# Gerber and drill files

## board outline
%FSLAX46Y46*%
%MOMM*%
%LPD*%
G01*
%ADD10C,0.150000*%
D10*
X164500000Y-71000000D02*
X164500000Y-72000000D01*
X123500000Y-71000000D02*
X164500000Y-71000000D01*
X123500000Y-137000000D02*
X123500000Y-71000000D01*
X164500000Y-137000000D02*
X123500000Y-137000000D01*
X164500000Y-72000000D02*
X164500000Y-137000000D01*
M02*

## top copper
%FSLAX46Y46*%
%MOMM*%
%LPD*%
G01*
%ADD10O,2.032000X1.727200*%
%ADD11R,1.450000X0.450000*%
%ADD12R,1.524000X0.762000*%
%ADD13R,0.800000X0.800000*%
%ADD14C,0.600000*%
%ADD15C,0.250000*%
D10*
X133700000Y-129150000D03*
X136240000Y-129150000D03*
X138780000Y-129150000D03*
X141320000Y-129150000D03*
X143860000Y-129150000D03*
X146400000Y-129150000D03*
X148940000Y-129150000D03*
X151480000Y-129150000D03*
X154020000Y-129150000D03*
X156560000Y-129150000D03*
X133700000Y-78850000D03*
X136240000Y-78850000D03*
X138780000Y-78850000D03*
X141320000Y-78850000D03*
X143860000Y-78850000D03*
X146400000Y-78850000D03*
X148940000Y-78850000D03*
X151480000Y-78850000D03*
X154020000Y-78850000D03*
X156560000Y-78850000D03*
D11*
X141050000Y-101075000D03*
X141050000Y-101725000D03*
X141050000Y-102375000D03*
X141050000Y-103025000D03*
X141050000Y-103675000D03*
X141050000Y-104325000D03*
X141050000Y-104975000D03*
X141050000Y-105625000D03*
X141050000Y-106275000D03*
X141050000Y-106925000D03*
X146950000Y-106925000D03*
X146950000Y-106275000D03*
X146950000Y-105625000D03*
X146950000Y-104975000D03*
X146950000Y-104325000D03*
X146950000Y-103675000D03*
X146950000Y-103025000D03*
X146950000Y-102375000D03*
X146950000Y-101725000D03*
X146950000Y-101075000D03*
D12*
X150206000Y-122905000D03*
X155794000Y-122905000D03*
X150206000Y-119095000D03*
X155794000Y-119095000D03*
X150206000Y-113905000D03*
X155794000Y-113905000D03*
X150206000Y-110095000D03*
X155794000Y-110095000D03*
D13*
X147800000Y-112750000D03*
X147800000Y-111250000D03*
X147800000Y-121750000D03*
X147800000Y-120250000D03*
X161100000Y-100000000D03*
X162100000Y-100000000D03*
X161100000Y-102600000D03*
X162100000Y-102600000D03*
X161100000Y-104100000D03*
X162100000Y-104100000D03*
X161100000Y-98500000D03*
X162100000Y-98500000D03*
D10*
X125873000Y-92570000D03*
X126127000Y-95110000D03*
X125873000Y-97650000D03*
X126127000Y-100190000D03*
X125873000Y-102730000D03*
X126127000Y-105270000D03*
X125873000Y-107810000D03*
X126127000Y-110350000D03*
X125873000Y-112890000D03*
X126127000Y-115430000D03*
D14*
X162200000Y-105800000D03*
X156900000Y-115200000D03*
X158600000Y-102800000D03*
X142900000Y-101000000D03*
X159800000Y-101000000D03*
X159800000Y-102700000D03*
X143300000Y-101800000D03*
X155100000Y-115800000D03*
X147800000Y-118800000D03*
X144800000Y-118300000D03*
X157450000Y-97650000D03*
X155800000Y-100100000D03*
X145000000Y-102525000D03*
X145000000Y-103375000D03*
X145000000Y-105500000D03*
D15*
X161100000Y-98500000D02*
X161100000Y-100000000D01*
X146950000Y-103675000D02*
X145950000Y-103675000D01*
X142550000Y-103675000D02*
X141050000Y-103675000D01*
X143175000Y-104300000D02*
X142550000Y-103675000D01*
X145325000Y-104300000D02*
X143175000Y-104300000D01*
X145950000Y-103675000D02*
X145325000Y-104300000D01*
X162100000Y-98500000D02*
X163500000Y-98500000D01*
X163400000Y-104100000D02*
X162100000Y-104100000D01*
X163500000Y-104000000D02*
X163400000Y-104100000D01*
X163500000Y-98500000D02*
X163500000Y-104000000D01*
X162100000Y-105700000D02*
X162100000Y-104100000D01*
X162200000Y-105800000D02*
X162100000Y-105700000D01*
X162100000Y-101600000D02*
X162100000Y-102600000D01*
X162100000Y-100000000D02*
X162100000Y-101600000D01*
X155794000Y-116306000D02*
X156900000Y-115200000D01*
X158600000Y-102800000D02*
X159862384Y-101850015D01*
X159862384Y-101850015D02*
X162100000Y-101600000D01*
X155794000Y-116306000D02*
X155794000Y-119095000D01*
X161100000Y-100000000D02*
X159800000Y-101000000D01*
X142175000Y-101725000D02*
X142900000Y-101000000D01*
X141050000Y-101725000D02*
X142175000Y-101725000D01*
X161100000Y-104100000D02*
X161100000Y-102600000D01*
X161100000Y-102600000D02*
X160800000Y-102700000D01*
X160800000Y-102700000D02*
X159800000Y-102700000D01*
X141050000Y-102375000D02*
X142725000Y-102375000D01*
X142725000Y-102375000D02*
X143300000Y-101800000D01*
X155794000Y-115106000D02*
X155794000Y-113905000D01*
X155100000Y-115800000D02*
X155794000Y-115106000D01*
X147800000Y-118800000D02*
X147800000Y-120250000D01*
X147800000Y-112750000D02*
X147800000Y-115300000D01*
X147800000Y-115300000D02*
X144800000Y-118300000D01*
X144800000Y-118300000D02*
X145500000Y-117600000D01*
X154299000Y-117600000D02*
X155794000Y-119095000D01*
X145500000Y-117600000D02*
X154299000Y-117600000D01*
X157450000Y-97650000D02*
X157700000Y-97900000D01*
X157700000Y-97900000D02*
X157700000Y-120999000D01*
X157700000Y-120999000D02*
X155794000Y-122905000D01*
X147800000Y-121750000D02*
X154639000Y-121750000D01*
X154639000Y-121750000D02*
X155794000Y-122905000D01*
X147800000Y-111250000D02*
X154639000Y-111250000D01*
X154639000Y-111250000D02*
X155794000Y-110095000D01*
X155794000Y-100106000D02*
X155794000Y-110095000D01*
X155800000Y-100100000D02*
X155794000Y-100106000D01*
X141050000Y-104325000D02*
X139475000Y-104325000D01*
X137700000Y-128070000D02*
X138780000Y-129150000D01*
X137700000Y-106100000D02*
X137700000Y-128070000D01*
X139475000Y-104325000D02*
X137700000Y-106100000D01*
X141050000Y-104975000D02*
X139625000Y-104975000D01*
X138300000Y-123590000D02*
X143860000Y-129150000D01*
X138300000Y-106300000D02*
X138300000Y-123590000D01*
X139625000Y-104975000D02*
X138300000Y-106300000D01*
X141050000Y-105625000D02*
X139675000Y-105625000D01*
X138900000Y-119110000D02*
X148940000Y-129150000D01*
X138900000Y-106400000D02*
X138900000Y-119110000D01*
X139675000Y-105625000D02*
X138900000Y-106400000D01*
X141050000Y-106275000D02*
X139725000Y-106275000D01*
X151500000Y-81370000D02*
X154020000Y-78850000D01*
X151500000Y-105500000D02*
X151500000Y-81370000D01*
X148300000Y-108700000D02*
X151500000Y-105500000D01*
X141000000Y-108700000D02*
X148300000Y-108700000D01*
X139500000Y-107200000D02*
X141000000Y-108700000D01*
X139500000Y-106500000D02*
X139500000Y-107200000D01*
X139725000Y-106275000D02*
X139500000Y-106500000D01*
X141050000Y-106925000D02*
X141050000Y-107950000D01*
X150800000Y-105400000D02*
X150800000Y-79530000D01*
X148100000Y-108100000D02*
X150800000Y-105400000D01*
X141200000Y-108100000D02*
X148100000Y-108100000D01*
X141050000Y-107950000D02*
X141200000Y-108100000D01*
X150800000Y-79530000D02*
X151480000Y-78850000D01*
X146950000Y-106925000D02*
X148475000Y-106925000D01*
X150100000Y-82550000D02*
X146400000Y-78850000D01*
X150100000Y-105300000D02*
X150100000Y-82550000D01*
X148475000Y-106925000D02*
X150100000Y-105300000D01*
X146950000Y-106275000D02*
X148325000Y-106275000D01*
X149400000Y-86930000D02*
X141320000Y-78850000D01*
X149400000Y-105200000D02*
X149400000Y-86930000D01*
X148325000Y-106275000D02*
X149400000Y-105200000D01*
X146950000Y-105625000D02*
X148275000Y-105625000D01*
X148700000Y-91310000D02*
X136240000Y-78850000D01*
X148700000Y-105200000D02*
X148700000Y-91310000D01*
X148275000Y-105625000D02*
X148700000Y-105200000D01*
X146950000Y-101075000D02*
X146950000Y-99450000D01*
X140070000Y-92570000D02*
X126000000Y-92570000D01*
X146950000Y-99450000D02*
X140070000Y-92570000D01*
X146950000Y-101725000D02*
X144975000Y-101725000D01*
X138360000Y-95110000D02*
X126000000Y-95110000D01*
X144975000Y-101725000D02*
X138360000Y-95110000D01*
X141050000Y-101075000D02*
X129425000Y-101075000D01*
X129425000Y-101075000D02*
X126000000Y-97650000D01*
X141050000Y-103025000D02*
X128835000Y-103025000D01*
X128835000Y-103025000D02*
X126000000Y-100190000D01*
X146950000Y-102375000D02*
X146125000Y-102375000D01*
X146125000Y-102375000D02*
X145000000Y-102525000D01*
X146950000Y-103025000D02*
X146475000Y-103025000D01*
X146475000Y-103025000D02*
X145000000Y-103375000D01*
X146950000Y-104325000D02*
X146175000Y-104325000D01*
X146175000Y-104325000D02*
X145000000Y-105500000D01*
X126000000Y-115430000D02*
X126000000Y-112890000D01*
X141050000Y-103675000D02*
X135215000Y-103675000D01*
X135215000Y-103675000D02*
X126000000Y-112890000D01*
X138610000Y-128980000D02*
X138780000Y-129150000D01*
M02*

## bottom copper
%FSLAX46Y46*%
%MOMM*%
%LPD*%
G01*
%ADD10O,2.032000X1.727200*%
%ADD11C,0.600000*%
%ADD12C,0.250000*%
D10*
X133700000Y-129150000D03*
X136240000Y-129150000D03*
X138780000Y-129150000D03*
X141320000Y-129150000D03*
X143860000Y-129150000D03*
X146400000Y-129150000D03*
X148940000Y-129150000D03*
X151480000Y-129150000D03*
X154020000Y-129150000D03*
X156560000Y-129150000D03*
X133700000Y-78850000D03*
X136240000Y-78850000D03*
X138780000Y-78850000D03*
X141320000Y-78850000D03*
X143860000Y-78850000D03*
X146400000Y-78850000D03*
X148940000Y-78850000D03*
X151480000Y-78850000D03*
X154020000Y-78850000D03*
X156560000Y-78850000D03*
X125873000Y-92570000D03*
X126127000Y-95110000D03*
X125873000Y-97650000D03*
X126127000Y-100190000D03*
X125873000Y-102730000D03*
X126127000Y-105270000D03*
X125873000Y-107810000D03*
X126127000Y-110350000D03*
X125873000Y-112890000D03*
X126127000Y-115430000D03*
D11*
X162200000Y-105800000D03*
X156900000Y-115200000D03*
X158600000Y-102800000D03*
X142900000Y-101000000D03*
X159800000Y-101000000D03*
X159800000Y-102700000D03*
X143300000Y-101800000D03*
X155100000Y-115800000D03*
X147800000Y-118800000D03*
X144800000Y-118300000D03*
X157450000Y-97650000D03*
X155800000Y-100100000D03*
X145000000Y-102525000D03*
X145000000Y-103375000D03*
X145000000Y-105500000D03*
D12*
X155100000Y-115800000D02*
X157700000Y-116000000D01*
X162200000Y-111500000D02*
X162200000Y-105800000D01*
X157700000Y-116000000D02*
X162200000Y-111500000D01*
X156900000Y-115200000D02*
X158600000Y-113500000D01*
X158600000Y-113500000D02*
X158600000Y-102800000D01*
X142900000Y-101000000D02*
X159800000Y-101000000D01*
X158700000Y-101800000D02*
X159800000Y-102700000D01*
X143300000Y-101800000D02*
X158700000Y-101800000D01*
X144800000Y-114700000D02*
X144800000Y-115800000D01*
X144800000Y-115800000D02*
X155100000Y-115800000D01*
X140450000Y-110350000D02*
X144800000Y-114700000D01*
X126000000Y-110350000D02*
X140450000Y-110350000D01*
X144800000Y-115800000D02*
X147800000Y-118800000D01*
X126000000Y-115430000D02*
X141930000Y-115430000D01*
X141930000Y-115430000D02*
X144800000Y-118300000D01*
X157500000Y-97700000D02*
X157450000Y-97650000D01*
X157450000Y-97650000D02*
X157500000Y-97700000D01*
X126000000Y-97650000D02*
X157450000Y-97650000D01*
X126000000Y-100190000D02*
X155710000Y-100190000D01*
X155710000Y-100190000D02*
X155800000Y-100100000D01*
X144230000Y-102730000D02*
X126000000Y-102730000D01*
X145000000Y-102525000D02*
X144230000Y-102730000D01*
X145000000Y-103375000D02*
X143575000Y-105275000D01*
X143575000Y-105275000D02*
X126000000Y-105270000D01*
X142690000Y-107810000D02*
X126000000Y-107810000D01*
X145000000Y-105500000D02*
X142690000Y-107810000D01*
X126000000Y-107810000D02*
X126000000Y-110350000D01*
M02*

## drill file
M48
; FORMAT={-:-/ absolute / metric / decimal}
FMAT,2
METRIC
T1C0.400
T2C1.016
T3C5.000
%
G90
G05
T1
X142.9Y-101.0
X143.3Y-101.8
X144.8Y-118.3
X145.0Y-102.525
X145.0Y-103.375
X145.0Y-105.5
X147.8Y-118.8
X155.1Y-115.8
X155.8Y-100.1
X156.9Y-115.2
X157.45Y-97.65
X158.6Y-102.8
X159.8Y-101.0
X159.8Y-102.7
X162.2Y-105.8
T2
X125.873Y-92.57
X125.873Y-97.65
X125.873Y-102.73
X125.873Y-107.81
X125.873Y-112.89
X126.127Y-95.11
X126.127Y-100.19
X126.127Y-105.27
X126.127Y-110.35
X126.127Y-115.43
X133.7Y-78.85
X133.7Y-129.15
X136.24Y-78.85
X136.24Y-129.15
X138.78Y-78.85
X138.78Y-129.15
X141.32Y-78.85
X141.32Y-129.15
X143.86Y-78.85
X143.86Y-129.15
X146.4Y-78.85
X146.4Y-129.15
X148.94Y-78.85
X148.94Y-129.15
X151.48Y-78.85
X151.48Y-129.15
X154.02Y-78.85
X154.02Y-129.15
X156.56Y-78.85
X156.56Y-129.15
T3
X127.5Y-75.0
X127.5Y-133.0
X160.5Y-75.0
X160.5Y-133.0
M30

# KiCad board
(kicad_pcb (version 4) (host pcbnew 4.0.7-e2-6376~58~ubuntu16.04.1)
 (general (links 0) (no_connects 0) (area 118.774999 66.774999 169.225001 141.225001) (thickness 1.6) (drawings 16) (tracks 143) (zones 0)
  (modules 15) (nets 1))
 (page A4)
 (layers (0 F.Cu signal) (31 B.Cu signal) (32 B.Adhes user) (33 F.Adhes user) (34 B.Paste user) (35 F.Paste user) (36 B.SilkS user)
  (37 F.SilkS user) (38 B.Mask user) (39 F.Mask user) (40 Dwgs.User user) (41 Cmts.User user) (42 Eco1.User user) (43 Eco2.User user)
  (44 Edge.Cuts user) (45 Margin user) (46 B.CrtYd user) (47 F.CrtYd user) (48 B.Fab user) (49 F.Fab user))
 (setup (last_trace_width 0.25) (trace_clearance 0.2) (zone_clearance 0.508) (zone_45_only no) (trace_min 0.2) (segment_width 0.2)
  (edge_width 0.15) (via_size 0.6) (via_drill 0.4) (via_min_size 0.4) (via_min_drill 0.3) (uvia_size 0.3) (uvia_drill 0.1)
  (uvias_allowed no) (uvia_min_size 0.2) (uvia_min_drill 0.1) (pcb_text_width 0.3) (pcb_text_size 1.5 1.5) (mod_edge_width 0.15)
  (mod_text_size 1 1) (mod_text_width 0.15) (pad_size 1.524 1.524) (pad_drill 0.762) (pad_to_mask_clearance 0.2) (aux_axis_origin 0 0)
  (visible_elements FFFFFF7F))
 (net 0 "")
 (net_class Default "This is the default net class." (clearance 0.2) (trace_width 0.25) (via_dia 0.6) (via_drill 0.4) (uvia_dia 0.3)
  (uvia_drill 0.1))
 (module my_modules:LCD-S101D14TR (layer B.Cu) (at 144 104 180)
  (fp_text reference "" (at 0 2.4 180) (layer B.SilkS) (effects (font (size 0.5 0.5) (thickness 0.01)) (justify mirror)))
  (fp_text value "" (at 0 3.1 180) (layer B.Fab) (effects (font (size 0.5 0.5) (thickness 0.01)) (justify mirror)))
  (pad 10 thru_hole oval (at 10.3 -25.15 180) (size 2.032 1.7272) (drill 1.016) (layers *.Cu *.Mask B.SilkS))
  (pad 9 thru_hole oval (at 7.76 -25.15 180) (size 2.032 1.7272) (drill 1.016) (layers *.Cu *.Mask B.SilkS))
  (pad 8 thru_hole oval (at 5.22 -25.15 180) (size 2.032 1.7272) (drill 1.016) (layers *.Cu *.Mask B.SilkS))
  (pad 7 thru_hole oval (at 2.68 -25.15 180) (size 2.032 1.7272) (drill 1.016) (layers *.Cu *.Mask B.SilkS))
  (pad 6 thru_hole oval (at 0.14 -25.15 180) (size 2.032 1.7272) (drill 1.016) (layers *.Cu *.Mask B.SilkS))
  (pad 5 thru_hole oval (at -2.4 -25.15 180) (size 2.032 1.7272) (drill 1.016) (layers *.Cu *.Mask B.SilkS))
  (pad 4 thru_hole oval (at -4.94 -25.15 180) (size 2.032 1.7272) (drill 1.016) (layers *.Cu *.Mask B.SilkS))
  (pad 3 thru_hole oval (at -7.48 -25.15 180) (size 2.032 1.7272) (drill 1.016) (layers *.Cu *.Mask B.SilkS))
  (pad 2 thru_hole oval (at -10.02 -25.15 180) (size 2.032 1.7272) (drill 1.016) (layers *.Cu *.Mask B.SilkS))
  (pad 1 thru_hole oval (at -12.56 -25.15 180) (size 2.032 1.7272) (drill 1.016) (layers *.Cu *.Mask B.SilkS))
  (pad 11 thru_hole oval (at 10.3 25.15 180) (size 2.032 1.7272) (drill 1.016) (layers *.Cu *.Mask B.SilkS))
  (pad 12 thru_hole oval (at 7.76 25.15 180) (size 2.032 1.7272) (drill 1.016) (layers *.Cu *.Mask B.SilkS))
  (pad 13 thru_hole oval (at 5.22 25.15 180) (size 2.032 1.7272) (drill 1.016) (layers *.Cu *.Mask B.SilkS))
  (pad 14 thru_hole oval (at 2.68 25.15 180) (size 2.032 1.7272) (drill 1.016) (layers *.Cu *.Mask B.SilkS))
  (pad 15 thru_hole oval (at 0.14 25.15 180) (size 2.032 1.7272) (drill 1.016) (layers *.Cu *.Mask B.SilkS))
  (pad 16 thru_hole oval (at -2.4 25.15 180) (size 2.032 1.7272) (drill 1.016) (layers *.Cu *.Mask B.SilkS))
  (pad 17 thru_hole oval (at -4.94 25.15 180) (size 2.032 1.7272) (drill 1.016) (layers *.Cu *.Mask B.SilkS))
  (pad 18 thru_hole oval (at -7.48 25.15 180) (size 2.032 1.7272) (drill 1.016) (layers *.Cu *.Mask B.SilkS))
  (pad 19 thru_hole oval (at -10.02 25.15 180) (size 2.032 1.7272) (drill 1.016) (layers *.Cu *.Mask B.SilkS))
  (pad 20 thru_hole oval (at -12.56 25.15 180) (size 2.032 1.7272) (drill 1.016) (layers *.Cu *.Mask B.SilkS)))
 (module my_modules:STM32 (layer F.Cu) (at 144 104)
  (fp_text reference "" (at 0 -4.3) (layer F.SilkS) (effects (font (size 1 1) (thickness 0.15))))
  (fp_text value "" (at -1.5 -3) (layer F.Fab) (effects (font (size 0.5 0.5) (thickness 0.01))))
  (pad BOOT smd rect (at -2.95 -2.925) (size 1.45 0.45) (layers F.Cu F.Paste F.Mask))
  (pad 2 smd rect (at -2.95 -2.275) (size 1.45 0.45) (layers F.Cu F.Paste F.Mask))
  (pad 3 smd rect (at -2.95 -1.625) (size 1.45 0.45) (layers F.Cu F.Paste F.Mask))
  (pad NRST smd rect (at -2.95 -0.975) (size 1.45 0.45) (layers F.Cu F.Paste F.Mask))
  (pad VCC smd rect (at -2.95 -0.325) (size 1.45 0.45) (layers F.Cu F.Paste F.Mask))
  (pad PA0 smd rect (at -2.95 0.325) (size 1.45 0.45) (layers F.Cu F.Paste F.Mask))
  (pad PA1 smd rect (at -2.95 0.975) (size 1.45 0.45) (layers F.Cu F.Paste F.Mask))
  (pad PA2 smd rect (at -2.95 1.625) (size 1.45 0.45) (layers F.Cu F.Paste F.Mask))
  (pad PA3 smd rect (at -2.95 2.275) (size 1.45 0.45) (layers F.Cu F.Paste F.Mask))
  (pad PA4 smd rect (at -2.95 2.925) (size 1.45 0.45) (layers F.Cu F.Paste F.Mask))
  (pad PA5 smd rect (at 2.95 2.925) (size 1.45 0.45) (layers F.Cu F.Paste F.Mask))
  (pad PA6 smd rect (at 2.95 2.275) (size 1.45 0.45) (layers F.Cu F.Paste F.Mask))
  (pad PA7 smd rect (at 2.95 1.625) (size 1.45 0.45) (layers F.Cu F.Paste F.Mask))
  (pad PB1 smd rect (at 2.95 0.975) (size 1.45 0.45) (layers F.Cu F.Paste F.Mask))
  (pad GND smd rect (at 2.95 0.325) (size 1.45 0.45) (layers F.Cu F.Paste F.Mask))
  (pad VCC smd rect (at 2.95 -0.325) (size 1.45 0.45) (layers F.Cu F.Paste F.Mask))
  (pad TX smd rect (at 2.95 -0.975) (size 1.45 0.45) (layers F.Cu F.Paste F.Mask))
  (pad RX smd rect (at 2.95 -1.625) (size 1.45 0.45) (layers F.Cu F.Paste F.Mask))
  (pad DIO smd rect (at 2.95 -2.275) (size 1.45 0.45) (layers F.Cu F.Paste F.Mask))
  (pad CLK smd rect (at 2.95 -2.925) (size 1.45 0.45) (layers F.Cu F.Paste F.Mask)))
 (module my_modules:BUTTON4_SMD (layer F.Cu) (at 153 121)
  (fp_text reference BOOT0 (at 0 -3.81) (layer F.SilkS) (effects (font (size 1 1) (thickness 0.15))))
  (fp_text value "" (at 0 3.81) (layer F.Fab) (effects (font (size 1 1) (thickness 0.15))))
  (pad 1 smd rect (at -2.794 1.905) (size 1.524 0.762) (layers F.Cu F.Paste F.Mask))
  (pad 2 smd rect (at 2.794 1.905) (size 1.524 0.762) (layers F.Cu F.Paste F.Mask))
  (pad 3 smd rect (at -2.794 -1.905) (size 1.524 0.762) (layers F.Cu F.Paste F.Mask))
  (pad 4 smd rect (at 2.794 -1.905) (size 1.524 0.762) (layers F.Cu F.Paste F.Mask)))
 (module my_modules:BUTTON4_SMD (layer F.Cu) (at 153 112)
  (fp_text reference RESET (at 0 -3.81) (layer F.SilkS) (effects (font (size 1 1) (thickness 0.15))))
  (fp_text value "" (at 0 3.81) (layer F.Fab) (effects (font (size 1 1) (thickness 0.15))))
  (pad 1 smd rect (at -2.794 1.905) (size 1.524 0.762) (layers F.Cu F.Paste F.Mask))
  (pad 2 smd rect (at 2.794 1.905) (size 1.524 0.762) (layers F.Cu F.Paste F.Mask))
  (pad 3 smd rect (at -2.794 -1.905) (size 1.524 0.762) (layers F.Cu F.Paste F.Mask))
  (pad 4 smd rect (at 2.794 -1.905) (size 1.524 0.762) (layers F.Cu F.Paste F.Mask)))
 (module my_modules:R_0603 (layer F.Cu) (at 147.8 112 90)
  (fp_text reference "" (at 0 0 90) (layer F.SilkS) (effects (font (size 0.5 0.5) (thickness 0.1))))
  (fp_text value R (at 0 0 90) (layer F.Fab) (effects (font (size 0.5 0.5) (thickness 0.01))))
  (pad 1 smd rect (at -0.75 0 90) (size 0.8 0.8) (layers F.Cu F.Paste F.Mask))
  (pad 2 smd rect (at 0.75 0 90) (size 0.8 0.8) (layers F.Cu F.Paste F.Mask)))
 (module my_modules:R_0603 (layer F.Cu) (at 147.8 121 90)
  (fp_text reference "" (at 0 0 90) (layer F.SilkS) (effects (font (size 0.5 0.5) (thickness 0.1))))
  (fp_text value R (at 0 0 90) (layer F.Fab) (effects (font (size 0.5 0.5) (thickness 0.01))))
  (pad 1 smd rect (at -0.75 0 90) (size 0.8 0.8) (layers F.Cu F.Paste F.Mask))
  (pad 2 smd rect (at 0.75 0 90) (size 0.8 0.8) (layers F.Cu F.Paste F.Mask)))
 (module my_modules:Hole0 (layer F.Cu) (at 160.5 133)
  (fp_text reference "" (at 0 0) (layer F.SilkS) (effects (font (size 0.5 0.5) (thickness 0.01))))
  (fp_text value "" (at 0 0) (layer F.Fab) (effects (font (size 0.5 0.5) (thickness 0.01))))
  (pad "" np_thru_hole circle (at 0 0) (size 5 5) (drill 5) (layers *.Cu *.Mask F.SilkS)))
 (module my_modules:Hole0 (layer F.Cu) (at 127.5 133)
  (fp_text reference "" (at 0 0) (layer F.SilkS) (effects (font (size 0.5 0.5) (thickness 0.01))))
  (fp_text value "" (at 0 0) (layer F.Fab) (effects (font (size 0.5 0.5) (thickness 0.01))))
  (pad "" np_thru_hole circle (at 0 0) (size 5 5) (drill 5) (layers *.Cu *.Mask F.SilkS)))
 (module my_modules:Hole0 (layer F.Cu) (at 160.5 75)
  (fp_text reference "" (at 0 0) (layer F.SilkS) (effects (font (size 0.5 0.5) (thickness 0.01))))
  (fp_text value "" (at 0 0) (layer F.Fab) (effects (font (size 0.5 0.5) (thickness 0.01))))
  (pad "" np_thru_hole circle (at 0 0) (size 5 5) (drill 5) (layers *.Cu *.Mask F.SilkS)))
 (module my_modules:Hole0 (layer F.Cu) (at 127.5 75)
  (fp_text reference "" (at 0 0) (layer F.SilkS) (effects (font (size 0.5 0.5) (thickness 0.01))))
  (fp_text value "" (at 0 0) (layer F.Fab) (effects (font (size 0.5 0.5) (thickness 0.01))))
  (pad "" np_thru_hole circle (at 0 0) (size 5 5) (drill 5) (layers *.Cu *.Mask F.SilkS)))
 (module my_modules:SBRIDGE (layer F.Cu) (at 161.6 100)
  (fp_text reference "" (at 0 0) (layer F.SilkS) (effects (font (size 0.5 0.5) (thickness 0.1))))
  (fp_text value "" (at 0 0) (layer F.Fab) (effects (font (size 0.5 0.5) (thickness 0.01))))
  (pad 1 smd rect (at -0.5 0) (size 0.8 0.8) (layers F.Cu F.Paste F.Mask))
  (pad 2 smd rect (at 0.5 0) (size 0.8 0.8) (layers F.Cu F.Paste F.Mask)))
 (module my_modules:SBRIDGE (layer F.Cu) (at 161.6 102.6)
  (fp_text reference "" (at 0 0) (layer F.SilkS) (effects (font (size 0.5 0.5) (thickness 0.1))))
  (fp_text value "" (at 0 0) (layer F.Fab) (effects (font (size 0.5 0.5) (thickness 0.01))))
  (pad 1 smd rect (at -0.5 0) (size 0.8 0.8) (layers F.Cu F.Paste F.Mask))
  (pad 2 smd rect (at 0.5 0) (size 0.8 0.8) (layers F.Cu F.Paste F.Mask)))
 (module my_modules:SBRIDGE (layer F.Cu) (at 161.6 104.1)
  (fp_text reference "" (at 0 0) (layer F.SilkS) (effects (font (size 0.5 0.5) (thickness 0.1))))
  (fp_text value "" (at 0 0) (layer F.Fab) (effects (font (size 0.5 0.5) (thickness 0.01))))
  (pad 1 smd rect (at -0.5 0) (size 0.8 0.8) (layers F.Cu F.Paste F.Mask))
  (pad 2 smd rect (at 0.5 0) (size 0.8 0.8) (layers F.Cu F.Paste F.Mask)))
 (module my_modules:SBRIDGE (layer F.Cu) (at 161.6 98.5)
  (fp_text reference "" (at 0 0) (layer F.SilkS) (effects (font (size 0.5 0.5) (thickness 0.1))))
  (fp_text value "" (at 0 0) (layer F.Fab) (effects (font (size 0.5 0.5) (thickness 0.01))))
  (pad 1 smd rect (at -0.5 0) (size 0.8 0.8) (layers F.Cu F.Paste F.Mask))
  (pad 2 smd rect (at 0.5 0) (size 0.8 0.8) (layers F.Cu F.Paste F.Mask)))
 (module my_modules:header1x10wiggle (layer F.Cu) (at 126 104)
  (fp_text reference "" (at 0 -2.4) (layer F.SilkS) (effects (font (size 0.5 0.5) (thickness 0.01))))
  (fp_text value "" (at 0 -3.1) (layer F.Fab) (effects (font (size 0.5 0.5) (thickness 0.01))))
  (pad 2 thru_hole oval (at -0.127 -11.43) (size 2.032 1.7272) (drill 1.016) (layers *.Cu *.Mask F.SilkS))
  (pad 3 thru_hole oval (at 0.127 -8.89) (size 2.032 1.7272) (drill 1.016) (layers *.Cu *.Mask F.SilkS))
  (pad 4 thru_hole oval (at -0.127 -6.35) (size 2.032 1.7272) (drill 1.016) (layers *.Cu *.Mask F.SilkS))
  (pad 5 thru_hole oval (at 0.127 -3.81) (size 2.032 1.7272) (drill 1.016) (layers *.Cu *.Mask F.SilkS))
  (pad 6 thru_hole oval (at -0.127 -1.27) (size 2.032 1.7272) (drill 1.016) (layers *.Cu *.Mask F.SilkS))
  (pad 7 thru_hole oval (at 0.127 1.27) (size 2.032 1.7272) (drill 1.016) (layers *.Cu *.Mask F.SilkS))
  (pad 8 thru_hole oval (at -0.127 3.81) (size 2.032 1.7272) (drill 1.016) (layers *.Cu *.Mask F.SilkS))
  (pad 9 thru_hole oval (at 0.127 6.35) (size 2.032 1.7272) (drill 1.016) (layers *.Cu *.Mask F.SilkS))
  (pad 10 thru_hole oval (at -0.127 8.89) (size 2.032 1.7272) (drill 1.016) (layers *.Cu *.Mask F.SilkS))
  (pad 11 thru_hole oval (at 0.127 11.43) (size 2.032 1.7272) (drill 1.016) (layers *.Cu *.Mask F.SilkS)))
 (gr_line (start 164.5 71) (end 164.5 72) (angle 90) (layer Edge.Cuts) (width 0.15))
 (gr_line (start 123.5 71) (end 164.5 71) (angle 90) (layer Edge.Cuts) (width 0.15))
 (gr_line (start 123.5 137) (end 123.5 71) (angle 90) (layer Edge.Cuts) (width 0.15))
 (gr_line (start 164.5 137) (end 123.5 137) (angle 90) (layer Edge.Cuts) (width 0.15))
 (gr_line (start 164.5 72) (end 164.5 137) (angle 90) (layer Edge.Cuts) (width 0.15))
 (segment (start 161.1 98.5) (end 161.1 100) (width 0.25) (layer F.Cu) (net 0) (status C00000))
 (segment (start 146.95 103.675) (end 145.95 103.675) (width 0.25) (layer F.Cu) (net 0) (status 400000))
 (segment (start 142.55 103.675) (end 141.05 103.675) (width 0.25) (layer F.Cu) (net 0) (status 800000))
 (segment (start 143.175 104.3) (end 142.55 103.675) (width 0.25) (layer F.Cu) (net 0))
 (segment (start 145.325 104.3) (end 143.175 104.3) (width 0.25) (layer F.Cu) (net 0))
 (segment (start 145.95 103.675) (end 145.325 104.3) (width 0.25) (layer F.Cu) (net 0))
 (segment (start 162.1 98.5) (end 163.5 98.5) (width 0.25) (layer F.Cu) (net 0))
 (segment (start 163.4 104.1) (end 162.1 104.1) (width 0.25) (layer F.Cu) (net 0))
 (segment (start 163.5 104) (end 163.4 104.1) (width 0.25) (layer F.Cu) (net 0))
 (segment (start 163.5 98.5) (end 163.5 104) (width 0.25) (layer F.Cu) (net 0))
 (segment (start 155.1 115.8) (end 157.7 116) (width 0.25) (layer B.Cu) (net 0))
 (segment (start 162.1 105.7) (end 162.1 104.1) (width 0.25) (layer F.Cu) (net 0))
 (segment (start 162.2 105.8) (end 162.1 105.7) (width 0.25) (layer F.Cu) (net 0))
 (via (at 162.2 105.8) (size 0.6) (drill 0.4) (layers F.Cu B.Cu) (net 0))
 (segment (start 162.2 111.5) (end 162.2 105.8) (width 0.25) (layer B.Cu) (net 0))
 (segment (start 157.7 116) (end 162.2 111.5) (width 0.25) (layer B.Cu) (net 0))
 (segment (start 162.1 101.6) (end 162.1 102.6) (width 0.25) (layer F.Cu) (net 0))
 (segment (start 162.1 100) (end 162.1 101.6) (width 0.25) (layer F.Cu) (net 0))
 (segment (start 155.794 116.306) (end 156.9 115.2) (width 0.25) (layer F.Cu) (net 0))
 (via (at 156.9 115.2) (size 0.6) (drill 0.4) (layers F.Cu B.Cu) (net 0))
 (segment (start 156.9 115.2) (end 158.6 113.5) (width 0.25) (layer B.Cu) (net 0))
 (segment (start 158.6 113.5) (end 158.6 102.8) (width 0.25) (layer B.Cu) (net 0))
 (via (at 158.6 102.8) (size 0.6) (drill 0.4) (layers F.Cu B.Cu) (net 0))
 (segment (start 158.6 102.8) (end 159.862384 101.850015) (width 0.25) (layer F.Cu) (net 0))
 (segment (start 159.862384 101.850015) (end 162.1 101.6) (width 0.25) (layer F.Cu) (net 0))
 (segment (start 155.794 116.306) (end 155.794 119.095) (width 0.25) (layer F.Cu) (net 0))
 (segment (start 161.1 100) (end 159.8 101) (width 0.25) (layer F.Cu) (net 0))
 (segment (start 142.175 101.725) (end 142.9 101) (width 0.25) (layer F.Cu) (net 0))
 (via (at 142.9 101) (size 0.6) (drill 0.4) (layers F.Cu B.Cu) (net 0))
 (segment (start 142.9 101) (end 159.8 101) (width 0.25) (layer B.Cu) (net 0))
 (via (at 159.8 101) (size 0.6) (drill 0.4) (layers F.Cu B.Cu) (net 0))
 (segment (start 141.05 101.725) (end 142.175 101.725) (width 0.25) (layer F.Cu) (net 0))
 (segment (start 161.1 104.1) (end 161.1 102.6) (width 0.25) (layer F.Cu) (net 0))
 (segment (start 161.1 102.6) (end 160.8 102.7) (width 0.25) (layer F.Cu) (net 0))
 (segment (start 160.8 102.7) (end 159.8 102.7) (width 0.25) (layer F.Cu) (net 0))
 (segment (start 141.05 102.375) (end 142.725 102.375) (width 0.25) (layer F.Cu) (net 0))
 (via (at 159.8 102.7) (size 0.6) (drill 0.4) (layers F.Cu B.Cu) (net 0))
 (segment (start 158.7 101.8) (end 159.8 102.7) (width 0.25) (layer B.Cu) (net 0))
 (segment (start 143.3 101.8) (end 158.7 101.8) (width 0.25) (layer B.Cu) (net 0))
 (via (at 143.3 101.8) (size 0.6) (drill 0.4) (layers F.Cu B.Cu) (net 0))
 (segment (start 142.725 102.375) (end 143.3 101.8) (width 0.25) (layer F.Cu) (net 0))
 (segment (start 144.8 114.7) (end 144.8 115.8) (width 0.25) (layer B.Cu) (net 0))
 (segment (start 144.8 115.8) (end 155.1 115.8) (width 0.25) (layer B.Cu) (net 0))
 (segment (start 155.794 115.106) (end 155.794 113.905) (width 0.25) (layer F.Cu) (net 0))
 (segment (start 155.1 115.8) (end 155.794 115.106) (width 0.25) (layer F.Cu) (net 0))
 (via (at 155.1 115.8) (size 0.6) (drill 0.4) (layers F.Cu B.Cu) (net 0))
 (segment (start 140.45 110.35) (end 144.8 114.7) (width 0.25) (layer B.Cu) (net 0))
 (segment (start 126 110.35) (end 140.45 110.35) (width 0.25) (layer B.Cu) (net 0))
 (segment (start 147.8 118.8) (end 147.8 120.25) (width 0.25) (layer F.Cu) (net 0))
 (via (at 147.8 118.8) (size 0.6) (drill 0.4) (layers F.Cu B.Cu) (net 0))
 (segment (start 144.8 115.8) (end 147.8 118.8) (width 0.25) (layer B.Cu) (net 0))
 (segment (start 147.8 112.75) (end 147.8 115.3) (width 0.25) (layer F.Cu) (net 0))
 (segment (start 147.8 115.3) (end 144.8 118.3) (width 0.25) (layer F.Cu) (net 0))
 (segment (start 144.8 118.3) (end 145.5 117.6) (width 0.25) (layer F.Cu) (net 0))
 (segment (start 126 115.43) (end 141.93 115.43) (width 0.25) (layer B.Cu) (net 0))
 (via (at 144.8 118.3) (size 0.6) (drill 0.4) (layers F.Cu B.Cu) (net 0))
 (segment (start 141.93 115.43) (end 144.8 118.3) (width 0.25) (layer B.Cu) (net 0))
 (segment (start 154.299 117.6) (end 155.794 119.095) (width 0.25) (layer F.Cu) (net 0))
 (segment (start 145.5 117.6) (end 154.299 117.6) (width 0.25) (layer F.Cu) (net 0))
 (segment (start 157.5 97.7) (end 157.45 97.65) (width 0.25) (layer B.Cu) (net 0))
 (segment (start 157.45 97.65) (end 157.5 97.7) (width 0.25) (layer B.Cu) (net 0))
 (via (at 157.45 97.65) (size 0.6) (drill 0.4) (layers F.Cu B.Cu) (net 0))
 (segment (start 157.45 97.65) (end 157.7 97.9) (width 0.25) (layer F.Cu) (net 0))
 (segment (start 157.7 97.9) (end 157.7 120.999) (width 0.25) (layer F.Cu) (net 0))
 (segment (start 157.7 120.999) (end 155.794 122.905) (width 0.25) (layer F.Cu) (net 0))
 (segment (start 126 97.65) (end 157.45 97.65) (width 0.25) (layer B.Cu) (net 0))
 (segment (start 147.8 121.75) (end 154.639 121.75) (width 0.25) (layer F.Cu) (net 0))
 (segment (start 154.639 121.75) (end 155.794 122.905) (width 0.25) (layer F.Cu) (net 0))
 (segment (start 147.8 111.25) (end 154.639 111.25) (width 0.25) (layer F.Cu) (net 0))
 (segment (start 154.639 111.25) (end 155.794 110.095) (width 0.25) (layer F.Cu) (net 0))
 (segment (start 126 100.19) (end 155.71 100.19) (width 0.25) (layer B.Cu) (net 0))
 (segment (start 155.794 100.106) (end 155.794 110.095) (width 0.25) (layer F.Cu) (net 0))
 (segment (start 155.8 100.1) (end 155.794 100.106) (width 0.25) (layer F.Cu) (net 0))
 (via (at 155.8 100.1) (size 0.6) (drill 0.4) (layers F.Cu B.Cu) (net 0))
 (segment (start 155.71 100.19) (end 155.8 100.1) (width 0.25) (layer B.Cu) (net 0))
 (segment (start 141.05 104.325) (end 139.475 104.325) (width 0.25) (layer F.Cu) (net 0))
 (segment (start 137.7 128.07) (end 138.78 129.15) (width 0.25) (layer F.Cu) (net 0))
 (segment (start 137.7 106.1) (end 137.7 128.07) (width 0.25) (layer F.Cu) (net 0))
 (segment (start 139.475 104.325) (end 137.7 106.1) (width 0.25) (layer F.Cu) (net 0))
 (segment (start 141.05 104.975) (end 139.625 104.975) (width 0.25) (layer F.Cu) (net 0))
 (segment (start 138.3 123.59) (end 143.86 129.15) (width 0.25) (layer F.Cu) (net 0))
 (segment (start 138.3 106.3) (end 138.3 123.59) (width 0.25) (layer F.Cu) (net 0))
 (segment (start 139.625 104.975) (end 138.3 106.3) (width 0.25) (layer F.Cu) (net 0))
 (segment (start 141.05 105.625) (end 139.675 105.625) (width 0.25) (layer F.Cu) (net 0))
 (segment (start 138.9 119.11) (end 148.94 129.15) (width 0.25) (layer F.Cu) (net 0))
 (segment (start 138.9 106.4) (end 138.9 119.11) (width 0.25) (layer F.Cu) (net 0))
 (segment (start 139.675 105.625) (end 138.9 106.4) (width 0.25) (layer F.Cu) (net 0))
 (segment (start 141.05 106.275) (end 139.725 106.275) (width 0.25) (layer F.Cu) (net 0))
 (segment (start 151.5 81.37) (end 154.02 78.85) (width 0.25) (layer F.Cu) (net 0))
 (segment (start 151.5 105.5) (end 151.5 81.37) (width 0.25) (layer F.Cu) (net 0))
 (segment (start 148.3 108.7) (end 151.5 105.5) (width 0.25) (layer F.Cu) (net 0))
 (segment (start 141 108.7) (end 148.3 108.7) (width 0.25) (layer F.Cu) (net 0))
 (segment (start 139.5 107.2) (end 141 108.7) (width 0.25) (layer F.Cu) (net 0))
 (segment (start 139.5 106.5) (end 139.5 107.2) (width 0.25) (layer F.Cu) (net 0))
 (segment (start 139.725 106.275) (end 139.5 106.5) (width 0.25) (layer F.Cu) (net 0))
 (segment (start 141.05 106.925) (end 141.05 107.95) (width 0.25) (layer F.Cu) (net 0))
 (segment (start 150.8 105.4) (end 150.8 79.53) (width 0.25) (layer F.Cu) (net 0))
 (segment (start 148.1 108.1) (end 150.8 105.4) (width 0.25) (layer F.Cu) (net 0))
 (segment (start 141.2 108.1) (end 148.1 108.1) (width 0.25) (layer F.Cu) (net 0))
 (segment (start 141.05 107.95) (end 141.2 108.1) (width 0.25) (layer F.Cu) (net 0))
 (segment (start 150.8 79.53) (end 151.48 78.85) (width 0.25) (layer F.Cu) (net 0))
 (segment (start 146.95 106.925) (end 148.475 106.925) (width 0.25) (layer F.Cu) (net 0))
 (segment (start 150.1 82.55) (end 146.4 78.85) (width 0.25) (layer F.Cu) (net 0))
 (segment (start 150.1 105.3) (end 150.1 82.55) (width 0.25) (layer F.Cu) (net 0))
 (segment (start 148.475 106.925) (end 150.1 105.3) (width 0.25) (layer F.Cu) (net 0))
 (segment (start 146.95 106.275) (end 148.325 106.275) (width 0.25) (layer F.Cu) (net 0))
 (segment (start 149.4 86.93) (end 141.32 78.85) (width 0.25) (layer F.Cu) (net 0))
 (segment (start 149.4 105.2) (end 149.4 86.93) (width 0.25) (layer F.Cu) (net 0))
 (segment (start 148.325 106.275) (end 149.4 105.2) (width 0.25) (layer F.Cu) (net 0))
 (segment (start 146.95 105.625) (end 148.275 105.625) (width 0.25) (layer F.Cu) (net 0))
 (segment (start 148.7 91.31) (end 136.24 78.85) (width 0.25) (layer F.Cu) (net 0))
 (segment (start 148.7 105.2) (end 148.7 91.31) (width 0.25) (layer F.Cu) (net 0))
 (segment (start 148.275 105.625) (end 148.7 105.2) (width 0.25) (layer F.Cu) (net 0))
 (segment (start 146.95 101.075) (end 146.95 99.45) (width 0.25) (layer F.Cu) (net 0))
 (segment (start 140.07 92.57) (end 126 92.57) (width 0.25) (layer F.Cu) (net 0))
 (segment (start 146.95 99.45) (end 140.07 92.57) (width 0.25) (layer F.Cu) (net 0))
 (segment (start 146.95 101.725) (end 144.975 101.725) (width 0.25) (layer F.Cu) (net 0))
 (segment (start 138.36 95.11) (end 126 95.11) (width 0.25) (layer F.Cu) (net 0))
 (segment (start 144.975 101.725) (end 138.36 95.11) (width 0.25) (layer F.Cu) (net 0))
 (segment (start 141.05 101.075) (end 129.425 101.075) (width 0.25) (layer F.Cu) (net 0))
 (segment (start 129.425 101.075) (end 126 97.65) (width 0.25) (layer F.Cu) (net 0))
 (segment (start 141.05 103.025) (end 128.835 103.025) (width 0.25) (layer F.Cu) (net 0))
 (segment (start 128.835 103.025) (end 126 100.19) (width 0.25) (layer F.Cu) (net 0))
 (segment (start 146.95 102.375) (end 146.125 102.375) (width 0.25) (layer F.Cu) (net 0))
 (segment (start 144.23 102.73) (end 126 102.73) (width 0.25) (layer B.Cu) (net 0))
 (segment (start 145 102.525) (end 144.23 102.73) (width 0.25) (layer B.Cu) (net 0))
 (via (at 145 102.525) (size 0.6) (drill 0.4) (layers F.Cu B.Cu) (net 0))
 (segment (start 146.125 102.375) (end 145 102.525) (width 0.25) (layer F.Cu) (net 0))
 (segment (start 146.95 103.025) (end 146.475 103.025) (width 0.25) (layer F.Cu) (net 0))
 (segment (start 146.475 103.025) (end 145 103.375) (width 0.25) (layer F.Cu) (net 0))
 (via (at 145 103.375) (size 0.6) (drill 0.4) (layers F.Cu B.Cu) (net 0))
 (segment (start 145 103.375) (end 143.575 105.275) (width 0.25) (layer B.Cu) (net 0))
 (segment (start 143.575 105.275) (end 126 105.27) (width 0.25) (layer B.Cu) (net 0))
 (segment (start 146.95 104.325) (end 146.175 104.325) (width 0.25) (layer F.Cu) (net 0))
 (segment (start 142.69 107.81) (end 126 107.81) (width 0.25) (layer B.Cu) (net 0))
 (segment (start 145 105.5) (end 142.69 107.81) (width 0.25) (layer B.Cu) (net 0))
 (via (at 145 105.5) (size 0.6) (drill 0.4) (layers F.Cu B.Cu) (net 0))
 (segment (start 146.175 104.325) (end 145 105.5) (width 0.25) (layer F.Cu) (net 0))
 (segment (start 126 107.81) (end 126 110.35) (width 0.25) (layer B.Cu) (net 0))
 (segment (start 126 115.43) (end 126 112.89) (width 0.25) (layer F.Cu) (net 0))
 (segment (start 141.05 103.675) (end 135.215 103.675) (width 0.25) (layer F.Cu) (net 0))
 (segment (start 135.215 103.675) (end 126 112.89) (width 0.25) (layer F.Cu) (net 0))
 (segment (start 138.61 128.98) (end 138.78 129.15) (width 0.25) (layer F.Cu) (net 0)))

